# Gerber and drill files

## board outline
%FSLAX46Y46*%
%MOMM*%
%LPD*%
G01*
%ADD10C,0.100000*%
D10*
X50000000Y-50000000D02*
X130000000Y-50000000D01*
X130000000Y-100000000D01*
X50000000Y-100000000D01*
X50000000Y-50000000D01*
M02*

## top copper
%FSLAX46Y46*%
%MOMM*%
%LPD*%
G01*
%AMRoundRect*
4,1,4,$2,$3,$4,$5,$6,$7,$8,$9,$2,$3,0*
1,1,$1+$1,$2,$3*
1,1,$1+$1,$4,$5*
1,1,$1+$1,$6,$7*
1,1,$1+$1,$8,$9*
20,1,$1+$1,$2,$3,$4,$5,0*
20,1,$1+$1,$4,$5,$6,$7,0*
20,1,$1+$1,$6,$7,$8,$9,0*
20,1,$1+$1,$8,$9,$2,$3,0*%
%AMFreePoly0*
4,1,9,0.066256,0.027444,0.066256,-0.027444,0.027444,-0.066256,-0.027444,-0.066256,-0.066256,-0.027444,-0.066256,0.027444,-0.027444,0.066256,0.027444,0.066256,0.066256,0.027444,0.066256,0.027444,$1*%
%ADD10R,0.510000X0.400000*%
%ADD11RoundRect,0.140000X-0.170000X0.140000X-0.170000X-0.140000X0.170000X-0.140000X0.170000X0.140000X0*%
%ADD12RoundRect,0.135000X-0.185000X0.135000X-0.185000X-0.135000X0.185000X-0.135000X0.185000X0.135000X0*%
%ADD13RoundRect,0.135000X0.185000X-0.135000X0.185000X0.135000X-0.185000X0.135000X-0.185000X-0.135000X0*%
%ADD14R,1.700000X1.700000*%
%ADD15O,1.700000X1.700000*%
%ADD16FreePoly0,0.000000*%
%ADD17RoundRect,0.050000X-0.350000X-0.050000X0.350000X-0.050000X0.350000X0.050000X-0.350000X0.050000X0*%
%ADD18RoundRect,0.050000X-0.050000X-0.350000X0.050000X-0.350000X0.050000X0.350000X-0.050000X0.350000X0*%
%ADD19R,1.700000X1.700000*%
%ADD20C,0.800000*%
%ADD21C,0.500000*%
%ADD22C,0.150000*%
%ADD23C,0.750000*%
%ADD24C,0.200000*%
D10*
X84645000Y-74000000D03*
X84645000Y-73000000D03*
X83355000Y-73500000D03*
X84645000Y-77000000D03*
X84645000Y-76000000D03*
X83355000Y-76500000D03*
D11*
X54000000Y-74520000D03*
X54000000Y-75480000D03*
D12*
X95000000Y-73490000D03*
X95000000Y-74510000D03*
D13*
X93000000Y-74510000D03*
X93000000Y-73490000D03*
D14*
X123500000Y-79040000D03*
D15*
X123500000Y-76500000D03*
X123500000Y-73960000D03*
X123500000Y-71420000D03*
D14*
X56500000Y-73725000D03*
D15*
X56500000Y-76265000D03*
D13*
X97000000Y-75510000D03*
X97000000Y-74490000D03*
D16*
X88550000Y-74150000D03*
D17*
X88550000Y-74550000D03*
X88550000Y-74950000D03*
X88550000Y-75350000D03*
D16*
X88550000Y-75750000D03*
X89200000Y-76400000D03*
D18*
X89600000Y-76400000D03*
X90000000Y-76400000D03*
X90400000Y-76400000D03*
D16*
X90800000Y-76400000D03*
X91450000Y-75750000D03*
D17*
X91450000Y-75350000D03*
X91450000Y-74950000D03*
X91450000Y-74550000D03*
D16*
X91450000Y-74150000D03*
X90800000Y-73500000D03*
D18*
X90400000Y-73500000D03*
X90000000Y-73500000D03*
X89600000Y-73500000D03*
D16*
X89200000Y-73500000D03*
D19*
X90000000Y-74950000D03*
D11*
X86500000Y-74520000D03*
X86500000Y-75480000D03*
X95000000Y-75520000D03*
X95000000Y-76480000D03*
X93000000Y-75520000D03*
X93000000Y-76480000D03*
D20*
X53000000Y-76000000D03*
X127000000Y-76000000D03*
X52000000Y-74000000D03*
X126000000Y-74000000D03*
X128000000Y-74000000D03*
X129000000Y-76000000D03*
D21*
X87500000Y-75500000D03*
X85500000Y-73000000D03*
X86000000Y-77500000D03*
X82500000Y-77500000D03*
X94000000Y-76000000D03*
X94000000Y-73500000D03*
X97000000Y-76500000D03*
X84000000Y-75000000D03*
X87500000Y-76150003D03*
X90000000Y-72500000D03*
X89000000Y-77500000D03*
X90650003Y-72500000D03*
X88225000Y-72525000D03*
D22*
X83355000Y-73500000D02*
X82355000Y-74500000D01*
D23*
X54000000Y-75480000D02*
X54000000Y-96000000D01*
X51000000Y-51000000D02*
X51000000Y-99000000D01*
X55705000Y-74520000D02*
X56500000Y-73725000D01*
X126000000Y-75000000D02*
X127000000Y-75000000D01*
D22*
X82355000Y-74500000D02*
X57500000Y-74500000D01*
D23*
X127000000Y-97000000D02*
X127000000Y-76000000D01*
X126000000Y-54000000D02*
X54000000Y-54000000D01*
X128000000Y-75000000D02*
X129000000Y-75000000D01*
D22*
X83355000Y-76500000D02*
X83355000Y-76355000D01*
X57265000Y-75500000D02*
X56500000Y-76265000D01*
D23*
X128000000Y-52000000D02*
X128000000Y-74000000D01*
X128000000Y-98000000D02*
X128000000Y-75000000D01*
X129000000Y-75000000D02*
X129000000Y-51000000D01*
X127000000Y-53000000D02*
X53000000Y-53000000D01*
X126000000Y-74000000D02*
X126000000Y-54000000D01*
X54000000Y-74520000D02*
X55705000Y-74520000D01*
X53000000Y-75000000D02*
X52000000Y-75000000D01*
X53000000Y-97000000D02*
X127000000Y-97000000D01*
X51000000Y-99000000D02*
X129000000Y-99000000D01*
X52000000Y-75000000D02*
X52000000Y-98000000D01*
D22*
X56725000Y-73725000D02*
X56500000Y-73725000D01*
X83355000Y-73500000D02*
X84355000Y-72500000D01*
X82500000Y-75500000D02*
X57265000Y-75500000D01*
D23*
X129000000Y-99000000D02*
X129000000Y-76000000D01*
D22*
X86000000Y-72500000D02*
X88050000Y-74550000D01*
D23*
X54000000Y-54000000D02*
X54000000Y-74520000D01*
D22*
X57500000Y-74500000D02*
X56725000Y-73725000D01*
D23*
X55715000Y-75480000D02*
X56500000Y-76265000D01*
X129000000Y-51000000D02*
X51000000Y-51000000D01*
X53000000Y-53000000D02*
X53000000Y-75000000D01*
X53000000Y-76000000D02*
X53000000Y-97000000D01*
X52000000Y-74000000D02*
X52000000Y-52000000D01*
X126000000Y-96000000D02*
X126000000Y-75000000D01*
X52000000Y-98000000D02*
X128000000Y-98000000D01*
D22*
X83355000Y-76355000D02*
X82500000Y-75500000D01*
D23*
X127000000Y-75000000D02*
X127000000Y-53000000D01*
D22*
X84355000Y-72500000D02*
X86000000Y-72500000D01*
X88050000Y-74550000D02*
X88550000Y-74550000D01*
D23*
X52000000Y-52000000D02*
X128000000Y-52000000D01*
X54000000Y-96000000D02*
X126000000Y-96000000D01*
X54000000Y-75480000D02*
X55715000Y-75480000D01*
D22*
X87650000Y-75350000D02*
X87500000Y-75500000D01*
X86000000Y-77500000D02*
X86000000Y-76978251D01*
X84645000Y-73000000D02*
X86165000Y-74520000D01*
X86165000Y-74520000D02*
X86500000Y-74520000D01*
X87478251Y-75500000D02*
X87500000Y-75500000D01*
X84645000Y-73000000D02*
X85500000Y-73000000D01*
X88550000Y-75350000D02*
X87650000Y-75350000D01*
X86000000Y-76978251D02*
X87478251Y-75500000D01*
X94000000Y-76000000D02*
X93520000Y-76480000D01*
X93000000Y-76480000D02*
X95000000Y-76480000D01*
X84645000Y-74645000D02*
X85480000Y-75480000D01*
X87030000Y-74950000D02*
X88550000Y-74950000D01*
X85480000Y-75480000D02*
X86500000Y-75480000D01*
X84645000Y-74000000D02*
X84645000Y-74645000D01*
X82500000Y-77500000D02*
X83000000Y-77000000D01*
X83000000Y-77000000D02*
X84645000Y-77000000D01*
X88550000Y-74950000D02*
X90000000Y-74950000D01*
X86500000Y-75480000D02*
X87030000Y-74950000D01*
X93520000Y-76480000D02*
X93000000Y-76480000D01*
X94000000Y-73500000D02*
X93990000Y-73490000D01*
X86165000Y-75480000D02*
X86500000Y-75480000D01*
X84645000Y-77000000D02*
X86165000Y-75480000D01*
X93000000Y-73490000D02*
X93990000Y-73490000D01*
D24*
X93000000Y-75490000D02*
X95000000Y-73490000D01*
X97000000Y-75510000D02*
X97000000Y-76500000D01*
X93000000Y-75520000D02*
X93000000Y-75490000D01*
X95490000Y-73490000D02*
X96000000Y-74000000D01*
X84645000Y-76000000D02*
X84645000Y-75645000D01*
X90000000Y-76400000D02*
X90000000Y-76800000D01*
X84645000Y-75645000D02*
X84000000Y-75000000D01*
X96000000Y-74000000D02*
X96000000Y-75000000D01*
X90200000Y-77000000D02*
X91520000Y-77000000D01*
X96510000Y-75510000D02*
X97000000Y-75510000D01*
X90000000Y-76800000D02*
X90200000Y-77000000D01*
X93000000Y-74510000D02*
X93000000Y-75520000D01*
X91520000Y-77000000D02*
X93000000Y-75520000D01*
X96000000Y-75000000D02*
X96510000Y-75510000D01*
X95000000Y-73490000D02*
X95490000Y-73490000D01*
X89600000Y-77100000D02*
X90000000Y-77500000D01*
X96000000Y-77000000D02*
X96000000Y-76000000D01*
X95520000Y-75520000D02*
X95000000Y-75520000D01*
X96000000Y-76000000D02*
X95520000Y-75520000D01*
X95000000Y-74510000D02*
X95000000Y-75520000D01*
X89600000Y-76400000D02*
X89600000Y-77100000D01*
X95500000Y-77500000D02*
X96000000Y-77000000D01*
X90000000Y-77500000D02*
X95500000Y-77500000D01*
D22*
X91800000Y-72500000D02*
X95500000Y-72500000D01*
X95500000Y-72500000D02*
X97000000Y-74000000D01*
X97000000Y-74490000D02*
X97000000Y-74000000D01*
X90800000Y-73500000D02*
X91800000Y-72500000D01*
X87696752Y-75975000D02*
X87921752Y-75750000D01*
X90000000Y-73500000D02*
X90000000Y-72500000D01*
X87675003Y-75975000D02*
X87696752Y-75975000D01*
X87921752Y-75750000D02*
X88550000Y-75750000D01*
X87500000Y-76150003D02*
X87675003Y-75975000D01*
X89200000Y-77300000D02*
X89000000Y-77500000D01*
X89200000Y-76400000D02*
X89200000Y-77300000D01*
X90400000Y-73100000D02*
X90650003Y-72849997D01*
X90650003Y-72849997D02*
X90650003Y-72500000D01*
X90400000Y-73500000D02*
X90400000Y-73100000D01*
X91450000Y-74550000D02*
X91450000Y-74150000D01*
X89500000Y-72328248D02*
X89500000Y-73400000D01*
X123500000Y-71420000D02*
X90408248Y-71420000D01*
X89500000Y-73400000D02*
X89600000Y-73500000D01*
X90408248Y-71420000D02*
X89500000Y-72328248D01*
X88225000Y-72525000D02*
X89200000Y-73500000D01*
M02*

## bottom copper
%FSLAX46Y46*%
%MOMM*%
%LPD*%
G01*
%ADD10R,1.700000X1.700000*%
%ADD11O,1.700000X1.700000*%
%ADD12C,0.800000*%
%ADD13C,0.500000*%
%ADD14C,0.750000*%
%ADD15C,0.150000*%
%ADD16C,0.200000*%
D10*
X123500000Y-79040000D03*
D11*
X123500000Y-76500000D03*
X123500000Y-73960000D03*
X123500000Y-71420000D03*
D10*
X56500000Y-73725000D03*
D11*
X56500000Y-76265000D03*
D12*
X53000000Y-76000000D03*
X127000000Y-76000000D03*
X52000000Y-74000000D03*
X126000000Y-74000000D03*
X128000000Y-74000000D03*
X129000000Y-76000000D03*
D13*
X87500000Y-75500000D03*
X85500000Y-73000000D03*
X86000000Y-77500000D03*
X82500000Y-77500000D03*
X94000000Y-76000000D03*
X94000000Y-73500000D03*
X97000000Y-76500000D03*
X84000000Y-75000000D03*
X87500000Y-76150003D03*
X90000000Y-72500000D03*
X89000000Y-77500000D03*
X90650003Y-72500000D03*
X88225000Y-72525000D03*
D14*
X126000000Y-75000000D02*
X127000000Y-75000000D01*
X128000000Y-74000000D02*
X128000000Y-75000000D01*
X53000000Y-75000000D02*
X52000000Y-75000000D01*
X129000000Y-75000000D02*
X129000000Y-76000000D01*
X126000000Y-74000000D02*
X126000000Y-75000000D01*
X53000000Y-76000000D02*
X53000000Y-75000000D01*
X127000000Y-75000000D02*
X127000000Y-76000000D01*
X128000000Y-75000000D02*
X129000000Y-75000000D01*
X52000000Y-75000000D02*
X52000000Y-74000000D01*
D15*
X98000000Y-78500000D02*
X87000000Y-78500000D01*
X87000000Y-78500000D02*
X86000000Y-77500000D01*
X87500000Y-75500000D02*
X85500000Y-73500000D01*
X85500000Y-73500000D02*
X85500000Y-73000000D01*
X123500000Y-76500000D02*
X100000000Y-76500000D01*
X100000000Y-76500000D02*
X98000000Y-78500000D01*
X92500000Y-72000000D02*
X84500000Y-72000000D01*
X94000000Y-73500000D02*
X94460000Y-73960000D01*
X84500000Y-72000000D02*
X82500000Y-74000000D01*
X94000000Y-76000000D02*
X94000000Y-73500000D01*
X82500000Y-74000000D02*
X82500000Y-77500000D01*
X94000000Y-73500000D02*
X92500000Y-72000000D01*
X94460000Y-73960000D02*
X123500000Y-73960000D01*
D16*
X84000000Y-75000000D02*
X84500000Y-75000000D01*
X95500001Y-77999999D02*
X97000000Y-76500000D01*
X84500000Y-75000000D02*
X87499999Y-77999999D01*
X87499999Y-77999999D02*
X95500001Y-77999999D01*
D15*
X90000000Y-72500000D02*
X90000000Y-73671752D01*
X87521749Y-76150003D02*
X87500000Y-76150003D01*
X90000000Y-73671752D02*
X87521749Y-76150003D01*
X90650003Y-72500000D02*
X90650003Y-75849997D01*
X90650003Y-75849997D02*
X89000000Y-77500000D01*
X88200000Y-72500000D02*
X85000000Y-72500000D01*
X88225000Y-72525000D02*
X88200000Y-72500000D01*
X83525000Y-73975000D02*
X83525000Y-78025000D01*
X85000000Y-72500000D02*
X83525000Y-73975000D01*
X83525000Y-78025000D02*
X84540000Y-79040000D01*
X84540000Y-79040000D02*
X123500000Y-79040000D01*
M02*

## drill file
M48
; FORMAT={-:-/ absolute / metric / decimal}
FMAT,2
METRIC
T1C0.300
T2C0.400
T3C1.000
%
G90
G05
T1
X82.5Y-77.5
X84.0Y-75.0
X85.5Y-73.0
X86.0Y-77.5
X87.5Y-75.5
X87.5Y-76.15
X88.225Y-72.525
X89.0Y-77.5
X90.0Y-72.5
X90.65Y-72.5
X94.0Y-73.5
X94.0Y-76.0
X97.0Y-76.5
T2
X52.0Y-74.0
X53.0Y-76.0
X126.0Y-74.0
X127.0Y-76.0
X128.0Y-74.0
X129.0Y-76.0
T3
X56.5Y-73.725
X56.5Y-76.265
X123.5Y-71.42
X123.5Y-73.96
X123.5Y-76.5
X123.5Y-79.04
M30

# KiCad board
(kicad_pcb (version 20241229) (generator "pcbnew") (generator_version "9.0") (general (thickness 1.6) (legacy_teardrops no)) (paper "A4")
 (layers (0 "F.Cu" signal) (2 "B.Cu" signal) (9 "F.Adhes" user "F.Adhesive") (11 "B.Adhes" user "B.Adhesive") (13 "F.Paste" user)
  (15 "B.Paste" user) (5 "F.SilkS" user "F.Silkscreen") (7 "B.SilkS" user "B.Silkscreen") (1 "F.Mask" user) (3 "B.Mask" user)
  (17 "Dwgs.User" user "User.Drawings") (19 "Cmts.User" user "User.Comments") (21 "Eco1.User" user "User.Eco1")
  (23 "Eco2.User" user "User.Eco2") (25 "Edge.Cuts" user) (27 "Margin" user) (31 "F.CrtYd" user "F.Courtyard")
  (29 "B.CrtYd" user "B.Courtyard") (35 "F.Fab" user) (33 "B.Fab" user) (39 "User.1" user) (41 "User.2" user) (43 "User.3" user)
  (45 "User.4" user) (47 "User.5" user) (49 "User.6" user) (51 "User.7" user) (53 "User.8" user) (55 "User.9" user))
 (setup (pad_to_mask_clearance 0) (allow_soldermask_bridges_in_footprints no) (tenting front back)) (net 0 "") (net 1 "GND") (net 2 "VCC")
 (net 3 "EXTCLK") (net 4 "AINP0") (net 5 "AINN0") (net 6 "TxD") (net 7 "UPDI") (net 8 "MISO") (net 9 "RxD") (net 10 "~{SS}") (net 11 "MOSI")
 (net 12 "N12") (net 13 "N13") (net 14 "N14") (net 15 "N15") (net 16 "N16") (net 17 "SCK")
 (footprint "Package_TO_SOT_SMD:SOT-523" (layer "F.Cu") (at 84 73.5 180)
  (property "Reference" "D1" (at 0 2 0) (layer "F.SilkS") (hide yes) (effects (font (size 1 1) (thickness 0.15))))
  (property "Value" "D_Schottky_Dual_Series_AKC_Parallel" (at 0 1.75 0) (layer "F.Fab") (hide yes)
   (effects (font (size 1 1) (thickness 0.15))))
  (pad "1" smd rect (at -0.645 -0.5) (size 0.51 0.4) (layers "F.Cu" "F.Mask" "F.Paste") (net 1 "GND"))
  (pad "2" smd rect (at -0.645 0.5) (size 0.51 0.4) (layers "F.Cu" "F.Mask" "F.Paste") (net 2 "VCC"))
  (pad "3" smd rect (at 0.645 0) (size 0.51 0.4) (layers "F.Cu" "F.Mask" "F.Paste") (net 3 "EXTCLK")))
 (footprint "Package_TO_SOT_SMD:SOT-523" (layer "F.Cu") (at 84 76.5 180)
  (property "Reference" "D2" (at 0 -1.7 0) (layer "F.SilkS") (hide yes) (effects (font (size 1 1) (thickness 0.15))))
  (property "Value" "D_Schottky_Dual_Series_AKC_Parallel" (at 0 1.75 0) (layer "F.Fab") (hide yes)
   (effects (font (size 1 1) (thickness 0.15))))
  (pad "1" smd rect (at -0.645 -0.5) (size 0.51 0.4) (layers "F.Cu" "F.Mask" "F.Paste") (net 1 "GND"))
  (pad "2" smd rect (at -0.645 0.5) (size 0.51 0.4) (layers "F.Cu" "F.Mask" "F.Paste") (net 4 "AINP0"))
  (pad "3" smd rect (at 0.645 0) (size 0.51 0.4) (layers "F.Cu" "F.Mask" "F.Paste") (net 3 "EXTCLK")))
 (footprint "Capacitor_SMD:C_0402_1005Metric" (layer "F.Cu") (at 54 75 -90)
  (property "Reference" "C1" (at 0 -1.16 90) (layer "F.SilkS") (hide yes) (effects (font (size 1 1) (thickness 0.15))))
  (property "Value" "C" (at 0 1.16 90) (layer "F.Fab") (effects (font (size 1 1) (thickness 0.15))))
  (pad "1" smd roundrect (at -0.48 0 270) (size 0.56 0.62) (layers "F.Cu" "F.Mask" "F.Paste") (roundrect_rratio 0.25) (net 3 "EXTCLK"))
  (pad "2" smd roundrect (at 0.48 0 270) (size 0.56 0.62) (layers "F.Cu" "F.Mask" "F.Paste") (roundrect_rratio 0.25) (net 3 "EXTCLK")))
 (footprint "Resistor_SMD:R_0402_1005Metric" (layer "F.Cu") (at 95 74 -90)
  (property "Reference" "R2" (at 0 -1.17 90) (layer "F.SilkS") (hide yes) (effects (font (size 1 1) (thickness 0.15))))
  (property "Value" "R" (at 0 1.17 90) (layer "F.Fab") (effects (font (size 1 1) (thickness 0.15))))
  (pad "1" smd roundrect (at -0.51 0 270) (size 0.54 0.64) (layers "F.Cu" "F.Mask" "F.Paste") (roundrect_rratio 0.25) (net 4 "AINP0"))
  (pad "2" smd roundrect (at 0.51 0 270) (size 0.54 0.64) (layers "F.Cu" "F.Mask" "F.Paste") (roundrect_rratio 0.25) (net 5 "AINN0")))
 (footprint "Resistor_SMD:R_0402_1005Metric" (layer "F.Cu") (at 93 74 90)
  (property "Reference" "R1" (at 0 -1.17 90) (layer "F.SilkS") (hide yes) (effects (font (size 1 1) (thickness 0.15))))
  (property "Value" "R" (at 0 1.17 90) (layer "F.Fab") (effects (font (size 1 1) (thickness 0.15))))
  (pad "1" smd roundrect (at -0.51 0 90) (size 0.54 0.64) (layers "F.Cu" "F.Mask" "F.Paste") (roundrect_rratio 0.25) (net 4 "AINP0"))
  (pad "2" smd roundrect (at 0.51 0 90) (size 0.54 0.64) (layers "F.Cu" "F.Mask" "F.Paste") (roundrect_rratio 0.25) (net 1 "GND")))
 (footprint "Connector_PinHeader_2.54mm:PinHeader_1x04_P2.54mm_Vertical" (layer "F.Cu") (at 123.5 79.04 180)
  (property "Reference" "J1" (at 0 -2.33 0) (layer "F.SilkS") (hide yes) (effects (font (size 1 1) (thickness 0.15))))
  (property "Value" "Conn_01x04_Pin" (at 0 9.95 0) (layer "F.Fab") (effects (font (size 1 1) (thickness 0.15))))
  (pad "1" thru_hole rect (at 0 0 180) (size 1.7 1.7) (drill 1) (layers "*.Cu" "*.Mask") (remove_unused_layers no) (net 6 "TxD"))
  (pad "2" thru_hole oval (at 0 2.54 180) (size 1.7 1.7) (drill 1) (layers "*.Cu" "*.Mask") (remove_unused_layers no) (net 2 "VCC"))
  (pad "3" thru_hole oval (at 0 5.08 180) (size 1.7 1.7) (drill 1) (layers "*.Cu" "*.Mask") (remove_unused_layers no) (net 1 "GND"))
  (pad "4" thru_hole oval (at 0 7.62 180) (size 1.7 1.7) (drill 1) (layers "*.Cu" "*.Mask") (remove_unused_layers no) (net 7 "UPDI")))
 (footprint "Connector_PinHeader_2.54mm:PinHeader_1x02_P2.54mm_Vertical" (layer "F.Cu") (at 56.5 73.725)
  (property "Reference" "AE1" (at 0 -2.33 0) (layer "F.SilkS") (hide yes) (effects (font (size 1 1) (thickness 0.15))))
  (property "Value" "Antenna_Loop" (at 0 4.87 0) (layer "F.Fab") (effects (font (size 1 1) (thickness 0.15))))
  (pad "1" thru_hole rect (at 0 0) (size 1.7 1.7) (drill 1) (layers "*.Cu" "*.Mask") (remove_unused_layers no) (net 3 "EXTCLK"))
  (pad "2" thru_hole oval (at 0 2.54) (size 1.7 1.7) (drill 1) (layers "*.Cu" "*.Mask") (remove_unused_layers no) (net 3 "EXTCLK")))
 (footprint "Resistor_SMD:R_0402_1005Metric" (layer "F.Cu") (at 97 75 90)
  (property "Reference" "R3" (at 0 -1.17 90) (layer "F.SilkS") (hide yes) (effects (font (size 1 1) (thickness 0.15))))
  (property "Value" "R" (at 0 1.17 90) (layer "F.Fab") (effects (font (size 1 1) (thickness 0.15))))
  (pad "1" smd roundrect (at -0.51 0 90) (size 0.54 0.64) (layers "F.Cu" "F.Mask" "F.Paste") (roundrect_rratio 0.25) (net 4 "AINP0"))
  (pad "2" smd roundrect (at 0.51 0 90) (size 0.54 0.64) (layers "F.Cu" "F.Mask" "F.Paste") (roundrect_rratio 0.25) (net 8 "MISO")))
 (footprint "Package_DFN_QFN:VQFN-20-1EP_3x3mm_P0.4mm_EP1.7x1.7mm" (layer "F.Cu") (at 90 74.95)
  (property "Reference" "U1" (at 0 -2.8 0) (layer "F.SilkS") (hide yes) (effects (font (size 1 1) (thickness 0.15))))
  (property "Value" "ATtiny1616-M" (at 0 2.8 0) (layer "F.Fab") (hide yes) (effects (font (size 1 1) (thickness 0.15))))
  (pad "" smd roundrect (at -0.425 -0.425) (size 0.69 0.69) (layers "F.Paste") (roundrect_rratio 0.25))
  (pad "" smd roundrect (at -0.425 0.425) (size 0.69 0.69) (layers "F.Paste") (roundrect_rratio 0.25))
  (pad "" smd roundrect (at 0.425 -0.425) (size 0.69 0.69) (layers "F.Paste") (roundrect_rratio 0.25))
  (pad "" smd roundrect (at 0.425 0.425) (size 0.69 0.69) (layers "F.Paste") (roundrect_rratio 0.25))
  (pad "1" smd custom (at -1.45 -0.8) (size 0.143431 0.143431) (layers "F.Cu" "F.Mask" "F.Paste") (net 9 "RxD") (thermal_bridge_angle 90)
   (options (clearance outline) (anchor circle)) (primitives))
  (pad "2" smd roundrect (at -1.45 -0.4) (size 0.8 0.2) (layers "F.Cu" "F.Mask" "F.Paste") (roundrect_rratio 0.25) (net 3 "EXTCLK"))
  (pad "3" smd roundrect (at -1.45 0) (size 0.8 0.2) (layers "F.Cu" "F.Mask" "F.Paste") (roundrect_rratio 0.25) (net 1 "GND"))
  (pad "4" smd roundrect (at -1.45 0.4) (size 0.8 0.2) (layers "F.Cu" "F.Mask" "F.Paste") (roundrect_rratio 0.25) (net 2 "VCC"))
  (pad "5" smd custom (at -1.45 0.8) (size 0.143431 0.143431) (layers "F.Cu" "F.Mask" "F.Paste") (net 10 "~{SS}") (thermal_bridge_angle 90)
   (options (clearance outline) (anchor circle)) (primitives))
  (pad "6" smd custom (at -0.8 1.45) (size 0.143431 0.143431) (layers "F.Cu" "F.Mask" "F.Paste") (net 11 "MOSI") (thermal_bridge_angle 90)
   (options (clearance outline) (anchor circle)) (primitives))
  (pad "7" smd roundrect (at -0.4 1.45) (size 0.2 0.8) (layers "F.Cu" "F.Mask" "F.Paste") (roundrect_rratio 0.25) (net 5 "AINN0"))
  (pad "8" smd roundrect (at 0 1.45) (size 0.2 0.8) (layers "F.Cu" "F.Mask" "F.Paste") (roundrect_rratio 0.25) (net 4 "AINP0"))
  (pad "9" smd roundrect (at 0.4 1.45) (size 0.2 0.8) (layers "F.Cu" "F.Mask" "F.Paste") (roundrect_rratio 0.25) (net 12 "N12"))
  (pad "10" smd custom (at 0.8 1.45) (size 0.143431 0.143431) (layers "F.Cu" "F.Mask" "F.Paste") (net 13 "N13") (thermal_bridge_angle 90)
   (options (clearance outline) (anchor circle)) (primitives))
  (pad "11" smd custom (at 1.45 0.8) (size 0.143431 0.143431) (layers "F.Cu" "F.Mask" "F.Paste") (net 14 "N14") (thermal_bridge_angle 90)
   (options (clearance outline) (anchor circle)) (primitives))
  (pad "12" smd roundrect (at 1.45 0.4) (size 0.8 0.2) (layers "F.Cu" "F.Mask" "F.Paste") (roundrect_rratio 0.25) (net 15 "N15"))
  (pad "13" smd roundrect (at 1.45 0) (size 0.8 0.2) (layers "F.Cu" "F.Mask" "F.Paste") (roundrect_rratio 0.25) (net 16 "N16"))
  (pad "14" smd roundrect (at 1.45 -0.4) (size 0.8 0.2) (layers "F.Cu" "F.Mask" "F.Paste") (roundrect_rratio 0.25) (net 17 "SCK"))
  (pad "15" smd custom (at 1.45 -0.8) (size 0.143431 0.143431) (layers "F.Cu" "F.Mask" "F.Paste") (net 17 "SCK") (thermal_bridge_angle 90)
   (options (clearance outline) (anchor circle)) (primitives))
  (pad "16" smd custom (at 0.8 -1.45) (size 0.143431 0.143431) (layers "F.Cu" "F.Mask" "F.Paste") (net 8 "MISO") (thermal_bridge_angle 90)
   (options (clearance outline) (anchor circle)) (primitives))
  (pad "17" smd roundrect (at 0.4 -1.45) (size 0.2 0.8) (layers "F.Cu" "F.Mask" "F.Paste") (roundrect_rratio 0.25) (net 11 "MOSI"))
  (pad "18" smd roundrect (at 0 -1.45) (size 0.2 0.8) (layers "F.Cu" "F.Mask" "F.Paste") (roundrect_rratio 0.25) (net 10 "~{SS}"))
  (pad "19" smd roundrect (at -0.4 -1.45) (size 0.2 0.8) (layers "F.Cu" "F.Mask" "F.Paste") (roundrect_rratio 0.25) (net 7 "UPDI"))
  (pad "20" smd custom (at -0.8 -1.45) (size 0.143431 0.143431) (layers "F.Cu" "F.Mask" "F.Paste") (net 6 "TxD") (thermal_bridge_angle 90)
   (options (clearance outline) (anchor circle)) (primitives))
  (pad "21" smd rect (at 0 0) (size 1.7 1.7) (layers "F.Cu" "F.Mask") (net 1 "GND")))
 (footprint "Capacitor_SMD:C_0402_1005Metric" (layer "F.Cu") (at 86.5 75 -90)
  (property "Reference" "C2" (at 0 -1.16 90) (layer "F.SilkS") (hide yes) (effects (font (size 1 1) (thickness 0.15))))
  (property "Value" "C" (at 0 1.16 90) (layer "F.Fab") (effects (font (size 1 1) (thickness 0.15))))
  (pad "1" smd roundrect (at -0.48 0 270) (size 0.56 0.62) (layers "F.Cu" "F.Mask" "F.Paste") (roundrect_rratio 0.25) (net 2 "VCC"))
  (pad "2" smd roundrect (at 0.48 0 270) (size 0.56 0.62) (layers "F.Cu" "F.Mask" "F.Paste") (roundrect_rratio 0.25) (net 1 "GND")))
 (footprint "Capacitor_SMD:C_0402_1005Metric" (layer "F.Cu") (at 95 76 -90)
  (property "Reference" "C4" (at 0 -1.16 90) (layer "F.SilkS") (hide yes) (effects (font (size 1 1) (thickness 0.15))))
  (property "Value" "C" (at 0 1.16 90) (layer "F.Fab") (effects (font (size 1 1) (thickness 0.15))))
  (pad "1" smd roundrect (at -0.48 0 270) (size 0.56 0.62) (layers "F.Cu" "F.Mask" "F.Paste") (roundrect_rratio 0.25) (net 5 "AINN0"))
  (pad "2" smd roundrect (at 0.48 0 270) (size 0.56 0.62) (layers "F.Cu" "F.Mask" "F.Paste") (roundrect_rratio 0.25) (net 1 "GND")))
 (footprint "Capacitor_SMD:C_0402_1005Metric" (layer "F.Cu") (at 93 76 -90)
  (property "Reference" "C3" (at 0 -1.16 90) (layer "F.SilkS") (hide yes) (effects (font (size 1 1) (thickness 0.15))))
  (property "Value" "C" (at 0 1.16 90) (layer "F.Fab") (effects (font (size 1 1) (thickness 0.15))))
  (pad "1" smd roundrect (at -0.48 0 270) (size 0.56 0.62) (layers "F.Cu" "F.Mask" "F.Paste") (roundrect_rratio 0.25) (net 4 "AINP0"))
  (pad "2" smd roundrect (at 0.48 0 270) (size 0.56 0.62) (layers "F.Cu" "F.Mask" "F.Paste") (roundrect_rratio 0.25) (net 1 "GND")))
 (gr_rect (start 50 50) (end 130 100) (stroke (width 0.1) (type default)) (fill no) (locked yes) (layer "Edge.Cuts"))
 (segment (start 83.355 73.5) (end 82.355 74.5) (width 0.15) (layer "F.Cu") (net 3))
 (segment (start 54 75.48) (end 54 96) (width 0.75) (layer "F.Cu") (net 3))
 (segment (start 51 51) (end 51 99) (width 0.75) (layer "F.Cu") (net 3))
 (segment (start 55.705 74.52) (end 56.5 73.725) (width 0.75) (layer "F.Cu") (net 3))
 (segment (start 126 75) (end 127 75) (width 0.75) (layer "F.Cu") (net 3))
 (segment (start 82.355 74.5) (end 57.5 74.5) (width 0.15) (layer "F.Cu") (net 3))
 (segment (start 127 97) (end 127 76) (width 0.75) (layer "F.Cu") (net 3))
 (segment (start 126 54) (end 54 54) (width 0.75) (layer "F.Cu") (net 3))
 (segment (start 128 75) (end 129 75) (width 0.75) (layer "F.Cu") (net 3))
 (segment (start 83.355 76.5) (end 83.355 76.355) (width 0.15) (layer "F.Cu") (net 3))
 (segment (start 57.265 75.5) (end 56.5 76.265) (width 0.15) (layer "F.Cu") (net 3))
 (segment (start 128 52) (end 128 74) (width 0.75) (layer "F.Cu") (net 3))
 (segment (start 128 98) (end 128 75) (width 0.75) (layer "F.Cu") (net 3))
 (segment (start 129 75) (end 129 51) (width 0.75) (layer "F.Cu") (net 3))
 (segment (start 127 53) (end 53 53) (width 0.75) (layer "F.Cu") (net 3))
 (segment (start 126 74) (end 126 54) (width 0.75) (layer "F.Cu") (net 3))
 (segment (start 54 74.52) (end 55.705 74.52) (width 0.75) (layer "F.Cu") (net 3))
 (segment (start 53 75) (end 52 75) (width 0.75) (layer "F.Cu") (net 3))
 (segment (start 53 97) (end 127 97) (width 0.75) (layer "F.Cu") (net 3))
 (segment (start 51 99) (end 129 99) (width 0.75) (layer "F.Cu") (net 3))
 (segment (start 52 75) (end 52 98) (width 0.75) (layer "F.Cu") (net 3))
 (segment (start 56.725 73.725) (end 56.5 73.725) (width 0.15) (layer "F.Cu") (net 3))
 (segment (start 83.355 73.5) (end 84.355 72.5) (width 0.15) (layer "F.Cu") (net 3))
 (segment (start 82.5 75.5) (end 57.265 75.5) (width 0.15) (layer "F.Cu") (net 3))
 (segment (start 129 99) (end 129 76) (width 0.75) (layer "F.Cu") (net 3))
 (segment (start 86 72.5) (end 88.05 74.55) (width 0.15) (layer "F.Cu") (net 3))
 (segment (start 54 54) (end 54 74.52) (width 0.75) (layer "F.Cu") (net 3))
 (segment (start 57.5 74.5) (end 56.725 73.725) (width 0.15) (layer "F.Cu") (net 3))
 (segment (start 55.715 75.48) (end 56.5 76.265) (width 0.75) (layer "F.Cu") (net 3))
 (segment (start 129 51) (end 51 51) (width 0.75) (layer "F.Cu") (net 3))
 (segment (start 53 53) (end 53 75) (width 0.75) (layer "F.Cu") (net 3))
 (segment (start 53 76) (end 53 97) (width 0.75) (layer "F.Cu") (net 3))
 (segment (start 52 74) (end 52 52) (width 0.75) (layer "F.Cu") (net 3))
 (segment (start 126 96) (end 126 75) (width 0.75) (layer "F.Cu") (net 3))
 (segment (start 52 98) (end 128 98) (width 0.75) (layer "F.Cu") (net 3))
 (segment (start 83.355 76.355) (end 82.5 75.5) (width 0.15) (layer "F.Cu") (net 3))
 (segment (start 127 75) (end 127 53) (width 0.75) (layer "F.Cu") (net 3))
 (segment (start 84.355 72.5) (end 86 72.5) (width 0.15) (layer "F.Cu") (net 3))
 (segment (start 88.05 74.55) (end 88.55 74.55) (width 0.15) (layer "F.Cu") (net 3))
 (segment (start 52 52) (end 128 52) (width 0.75) (layer "F.Cu") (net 3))
 (segment (start 54 96) (end 126 96) (width 0.75) (layer "F.Cu") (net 3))
 (segment (start 54 75.48) (end 55.715 75.48) (width 0.75) (layer "F.Cu") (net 3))
 (via (at 53 76) (size 0.8) (drill 0.4) (layers "F.Cu" "B.Cu") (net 3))
 (via (at 127 76) (size 0.8) (drill 0.4) (layers "F.Cu" "B.Cu") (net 3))
 (via (at 52 74) (size 0.8) (drill 0.4) (layers "F.Cu" "B.Cu") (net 3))
 (via (at 126 74) (size 0.8) (drill 0.4) (layers "F.Cu" "B.Cu") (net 3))
 (via (at 128 74) (size 0.8) (drill 0.4) (layers "F.Cu" "B.Cu") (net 3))
 (via (at 129 76) (size 0.8) (drill 0.4) (layers "F.Cu" "B.Cu") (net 3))
 (segment (start 126 75) (end 127 75) (width 0.75) (layer "B.Cu") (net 3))
 (segment (start 128 74) (end 128 75) (width 0.75) (layer "B.Cu") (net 3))
 (segment (start 53 75) (end 52 75) (width 0.75) (layer "B.Cu") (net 3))
 (segment (start 129 75) (end 129 76) (width 0.75) (layer "B.Cu") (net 3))
 (segment (start 126 74) (end 126 75) (width 0.75) (layer "B.Cu") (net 3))
 (segment (start 53 76) (end 53 75) (width 0.75) (layer "B.Cu") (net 3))
 (segment (start 127 75) (end 127 76) (width 0.75) (layer "B.Cu") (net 3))
 (segment (start 128 75) (end 129 75) (width 0.75) (layer "B.Cu") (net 3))
 (segment (start 52 75) (end 52 74) (width 0.75) (layer "B.Cu") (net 3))
 (segment (start 87.65 75.35) (end 87.5 75.5) (width 0.15) (layer "F.Cu") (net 2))
 (segment (start 86 77.5) (end 86 76.978251) (width 0.15) (layer "F.Cu") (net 2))
 (segment (start 84.645 73) (end 86.165 74.52) (width 0.15) (layer "F.Cu") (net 2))
 (segment (start 86.165 74.52) (end 86.5 74.52) (width 0.15) (layer "F.Cu") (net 2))
 (segment (start 87.478251 75.5) (end 87.5 75.5) (width 0.15) (layer "F.Cu") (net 2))
 (segment (start 84.645 73) (end 85.5 73) (width 0.15) (layer "F.Cu") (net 2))
 (segment (start 88.55 75.35) (end 87.65 75.35) (width 0.15) (layer "F.Cu") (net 2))
 (segment (start 86 76.978251) (end 87.478251 75.5) (width 0.15) (layer "F.Cu") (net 2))
 (via (at 87.5 75.5) (size 0.5) (drill 0.3) (layers "F.Cu" "B.Cu") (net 2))
 (via (at 85.5 73) (size 0.5) (drill 0.3) (layers "F.Cu" "B.Cu") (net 2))
 (via (at 86 77.5) (size 0.5) (drill 0.3) (layers "F.Cu" "B.Cu") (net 2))
 (segment (start 98 78.5) (end 87 78.5) (width 0.15) (layer "B.Cu") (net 2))
 (segment (start 87 78.5) (end 86 77.5) (width 0.15) (layer "B.Cu") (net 2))
 (segment (start 87.5 75.5) (end 85.5 73.5) (width 0.15) (layer "B.Cu") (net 2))
 (segment (start 85.5 73.5) (end 85.5 73) (width 0.15) (layer "B.Cu") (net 2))
 (segment (start 123.5 76.5) (end 100 76.5) (width 0.15) (layer "B.Cu") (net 2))
 (segment (start 100 76.5) (end 98 78.5) (width 0.15) (layer "B.Cu") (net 2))
 (segment (start 94 76) (end 93.52 76.48) (width 0.15) (layer "F.Cu") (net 1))
 (segment (start 93 76.48) (end 95 76.48) (width 0.15) (layer "F.Cu") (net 1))
 (segment (start 84.645 74.645) (end 85.48 75.48) (width 0.15) (layer "F.Cu") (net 1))
 (segment (start 87.03 74.95) (end 88.55 74.95) (width 0.15) (layer "F.Cu") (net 1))
 (segment (start 85.48 75.48) (end 86.5 75.48) (width 0.15) (layer "F.Cu") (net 1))
 (segment (start 84.645 74) (end 84.645 74.645) (width 0.15) (layer "F.Cu") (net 1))
 (segment (start 82.5 77.5) (end 83 77) (width 0.15) (layer "F.Cu") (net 1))
 (segment (start 83 77) (end 84.645 77) (width 0.15) (layer "F.Cu") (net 1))
 (segment (start 88.55 74.95) (end 90 74.95) (width 0.15) (layer "F.Cu") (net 1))
 (segment (start 86.5 75.48) (end 87.03 74.95) (width 0.15) (layer "F.Cu") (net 1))
 (segment (start 93.52 76.48) (end 93 76.48) (width 0.15) (layer "F.Cu") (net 1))
 (segment (start 94 73.5) (end 93.99 73.49) (width 0.15) (layer "F.Cu") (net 1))
 (segment (start 86.165 75.48) (end 86.5 75.48) (width 0.15) (layer "F.Cu") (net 1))
 (segment (start 84.645 77) (end 86.165 75.48) (width 0.15) (layer "F.Cu") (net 1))
 (segment (start 93 73.49) (end 93.99 73.49) (width 0.15) (layer "F.Cu") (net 1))
 (via (at 82.5 77.5) (size 0.5) (drill 0.3) (layers "F.Cu" "B.Cu") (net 1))
 (via (at 94 76) (size 0.5) (drill 0.3) (layers "F.Cu" "B.Cu") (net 1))
 (via (at 94 73.5) (size 0.5) (drill 0.3) (layers "F.Cu" "B.Cu") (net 1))
 (segment (start 92.5 72) (end 84.5 72) (width 0.15) (layer "B.Cu") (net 1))
 (segment (start 94 73.5) (end 94.46 73.96) (width 0.15) (layer "B.Cu") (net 1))
 (segment (start 84.5 72) (end 82.5 74) (width 0.15) (layer "B.Cu") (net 1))
 (segment (start 94 76) (end 94 73.5) (width 0.15) (layer "B.Cu") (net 1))
 (segment (start 82.5 74) (end 82.5 77.5) (width 0.15) (layer "B.Cu") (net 1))
 (segment (start 94 73.5) (end 92.5 72) (width 0.15) (layer "B.Cu") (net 1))
 (segment (start 94.46 73.96) (end 123.5 73.96) (width 0.15) (layer "B.Cu") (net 1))
 (segment (start 93 75.49) (end 95 73.49) (width 0.2) (layer "F.Cu") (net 4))
 (segment (start 97 75.51) (end 97 76.5) (width 0.2) (layer "F.Cu") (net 4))
 (segment (start 93 75.52) (end 93 75.49) (width 0.2) (layer "F.Cu") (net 4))
 (segment (start 95.49 73.49) (end 96 74) (width 0.2) (layer "F.Cu") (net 4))
 (segment (start 84.645 76) (end 84.645 75.645) (width 0.2) (layer "F.Cu") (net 4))
 (segment (start 90 76.4) (end 90 76.8) (width 0.2) (layer "F.Cu") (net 4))
 (segment (start 84.645 75.645) (end 84 75) (width 0.2) (layer "F.Cu") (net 4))
 (segment (start 96 74) (end 96 75) (width 0.2) (layer "F.Cu") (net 4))
 (segment (start 90.2 77) (end 91.52 77) (width 0.2) (layer "F.Cu") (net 4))
 (segment (start 96.51 75.51) (end 97 75.51) (width 0.2) (layer "F.Cu") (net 4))
 (segment (start 90 76.8) (end 90.2 77) (width 0.2) (layer "F.Cu") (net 4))
 (segment (start 93 74.51) (end 93 75.52) (width 0.2) (layer "F.Cu") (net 4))
 (segment (start 91.52 77) (end 93 75.52) (width 0.2) (layer "F.Cu") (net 4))
 (segment (start 96 75) (end 96.51 75.51) (width 0.2) (layer "F.Cu") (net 4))
 (segment (start 95 73.49) (end 95.49 73.49) (width 0.2) (layer "F.Cu") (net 4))
 (via (at 97 76.5) (size 0.5) (drill 0.3) (layers "F.Cu" "B.Cu") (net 4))
 (via (at 84 75) (size 0.5) (drill 0.3) (layers "F.Cu" "B.Cu") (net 4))
 (segment (start 84 75) (end 84.5 75) (width 0.2) (layer "B.Cu") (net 4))
 (segment (start 95.500001 77.999999) (end 97 76.5) (width 0.2) (layer "B.Cu") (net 4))
 (segment (start 84.5 75) (end 87.499999 77.999999) (width 0.2) (layer "B.Cu") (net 4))
 (segment (start 87.499999 77.999999) (end 95.500001 77.999999) (width 0.2) (layer "B.Cu") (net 4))
 (segment (start 89.6 77.1) (end 90 77.5) (width 0.2) (layer "F.Cu") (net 5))
 (segment (start 96 77) (end 96 76) (width 0.2) (layer "F.Cu") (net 5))
 (segment (start 95.52 75.52) (end 95 75.52) (width 0.2) (layer "F.Cu") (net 5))
 (segment (start 96 76) (end 95.52 75.52) (width 0.2) (layer "F.Cu") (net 5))
 (segment (start 95 74.51) (end 95 75.52) (width 0.2) (layer "F.Cu") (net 5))
 (segment (start 89.6 76.4) (end 89.6 77.1) (width 0.2) (layer "F.Cu") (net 5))
 (segment (start 95.5 77.5) (end 96 77) (width 0.2) (layer "F.Cu") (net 5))
 (segment (start 90 77.5) (end 95.5 77.5) (width 0.2) (layer "F.Cu") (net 5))
 (segment (start 91.8 72.5) (end 95.5 72.5) (width 0.15) (layer "F.Cu") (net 8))
 (segment (start 95.5 72.5) (end 97 74) (width 0.15) (layer "F.Cu") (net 8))
 (segment (start 97 74.49) (end 97 74) (width 0.15) (layer "F.Cu") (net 8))
 (segment (start 90.8 73.5) (end 91.8 72.5) (width 0.15) (layer "F.Cu") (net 8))
 (segment (start 87.696752 75.975) (end 87.921752 75.75) (width 0.15) (layer "F.Cu") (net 10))
 (segment (start 90 73.5) (end 90 72.5) (width 0.15) (layer "F.Cu") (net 10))
 (segment (start 87.675003 75.975) (end 87.696752 75.975) (width 0.15) (layer "F.Cu") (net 10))
 (segment (start 87.921752 75.75) (end 88.55 75.75) (width 0.15) (layer "F.Cu") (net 10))
 (segment (start 87.5 76.150003) (end 87.675003 75.975) (width 0.15) (layer "F.Cu") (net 10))
 (via (at 87.5 76.150003) (size 0.5) (drill 0.3) (layers "F.Cu" "B.Cu") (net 10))
 (via (at 90 72.5) (size 0.5) (drill 0.3) (layers "F.Cu" "B.Cu") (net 10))
 (segment (start 90 72.5) (end 90 73.671752) (width 0.15) (layer "B.Cu") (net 10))
 (segment (start 87.521749 76.150003) (end 87.5 76.150003) (width 0.15) (layer "B.Cu") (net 10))
 (segment (start 90 73.671752) (end 87.521749 76.150003) (width 0.15) (layer "B.Cu") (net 10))
 (segment (start 89.2 77.3) (end 89 77.5) (width 0.15) (layer "F.Cu") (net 11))
 (segment (start 89.2 76.4) (end 89.2 77.3) (width 0.15) (layer "F.Cu") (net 11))
 (segment (start 90.4 73.1) (end 90.650003 72.849997) (width 0.15) (layer "F.Cu") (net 11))
 (segment (start 90.650003 72.849997) (end 90.650003 72.5) (width 0.15) (layer "F.Cu") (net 11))
 (segment (start 90.4 73.5) (end 90.4 73.1) (width 0.15) (layer "F.Cu") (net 11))
 (via (at 89 77.5) (size 0.5) (drill 0.3) (layers "F.Cu" "B.Cu") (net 11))
 (via (at 90.650003 72.5) (size 0.5) (drill 0.3) (layers "F.Cu" "B.Cu") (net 11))
 (segment (start 90.650003 72.5) (end 90.650003 75.849997) (width 0.15) (layer "B.Cu") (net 11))
 (segment (start 90.650003 75.849997) (end 89 77.5) (width 0.15) (layer "B.Cu") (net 11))
 (segment (start 91.45 74.55) (end 91.45 74.15) (width 0.15) (layer "F.Cu") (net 17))
 (segment (start 89.5 72.328248) (end 89.5 73.4) (width 0.15) (layer "F.Cu") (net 7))
 (segment (start 123.5 71.42) (end 90.408248 71.42) (width 0.15) (layer "F.Cu") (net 7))
 (segment (start 89.5 73.4) (end 89.6 73.5) (width 0.15) (layer "F.Cu") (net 7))
 (segment (start 90.408248 71.42) (end 89.5 72.328248) (width 0.15) (layer "F.Cu") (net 7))
 (segment (start 88.225 72.525) (end 89.2 73.5) (width 0.15) (layer "F.Cu") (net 6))
 (via (at 88.225 72.525) (size 0.5) (drill 0.3) (layers "F.Cu" "B.Cu") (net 6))
 (segment (start 88.2 72.5) (end 85 72.5) (width 0.15) (layer "B.Cu") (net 6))
 (segment (start 88.225 72.525) (end 88.2 72.5) (width 0.15) (layer "B.Cu") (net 6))
 (segment (start 83.525 73.975) (end 83.525 78.025) (width 0.15) (layer "B.Cu") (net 6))
 (segment (start 85 72.5) (end 83.525 73.975) (width 0.15) (layer "B.Cu") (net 6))
 (segment (start 83.525 78.025) (end 84.54 79.04) (width 0.15) (layer "B.Cu") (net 6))
 (segment (start 84.54 79.04) (end 123.5 79.04) (width 0.15) (layer "B.Cu") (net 6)))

